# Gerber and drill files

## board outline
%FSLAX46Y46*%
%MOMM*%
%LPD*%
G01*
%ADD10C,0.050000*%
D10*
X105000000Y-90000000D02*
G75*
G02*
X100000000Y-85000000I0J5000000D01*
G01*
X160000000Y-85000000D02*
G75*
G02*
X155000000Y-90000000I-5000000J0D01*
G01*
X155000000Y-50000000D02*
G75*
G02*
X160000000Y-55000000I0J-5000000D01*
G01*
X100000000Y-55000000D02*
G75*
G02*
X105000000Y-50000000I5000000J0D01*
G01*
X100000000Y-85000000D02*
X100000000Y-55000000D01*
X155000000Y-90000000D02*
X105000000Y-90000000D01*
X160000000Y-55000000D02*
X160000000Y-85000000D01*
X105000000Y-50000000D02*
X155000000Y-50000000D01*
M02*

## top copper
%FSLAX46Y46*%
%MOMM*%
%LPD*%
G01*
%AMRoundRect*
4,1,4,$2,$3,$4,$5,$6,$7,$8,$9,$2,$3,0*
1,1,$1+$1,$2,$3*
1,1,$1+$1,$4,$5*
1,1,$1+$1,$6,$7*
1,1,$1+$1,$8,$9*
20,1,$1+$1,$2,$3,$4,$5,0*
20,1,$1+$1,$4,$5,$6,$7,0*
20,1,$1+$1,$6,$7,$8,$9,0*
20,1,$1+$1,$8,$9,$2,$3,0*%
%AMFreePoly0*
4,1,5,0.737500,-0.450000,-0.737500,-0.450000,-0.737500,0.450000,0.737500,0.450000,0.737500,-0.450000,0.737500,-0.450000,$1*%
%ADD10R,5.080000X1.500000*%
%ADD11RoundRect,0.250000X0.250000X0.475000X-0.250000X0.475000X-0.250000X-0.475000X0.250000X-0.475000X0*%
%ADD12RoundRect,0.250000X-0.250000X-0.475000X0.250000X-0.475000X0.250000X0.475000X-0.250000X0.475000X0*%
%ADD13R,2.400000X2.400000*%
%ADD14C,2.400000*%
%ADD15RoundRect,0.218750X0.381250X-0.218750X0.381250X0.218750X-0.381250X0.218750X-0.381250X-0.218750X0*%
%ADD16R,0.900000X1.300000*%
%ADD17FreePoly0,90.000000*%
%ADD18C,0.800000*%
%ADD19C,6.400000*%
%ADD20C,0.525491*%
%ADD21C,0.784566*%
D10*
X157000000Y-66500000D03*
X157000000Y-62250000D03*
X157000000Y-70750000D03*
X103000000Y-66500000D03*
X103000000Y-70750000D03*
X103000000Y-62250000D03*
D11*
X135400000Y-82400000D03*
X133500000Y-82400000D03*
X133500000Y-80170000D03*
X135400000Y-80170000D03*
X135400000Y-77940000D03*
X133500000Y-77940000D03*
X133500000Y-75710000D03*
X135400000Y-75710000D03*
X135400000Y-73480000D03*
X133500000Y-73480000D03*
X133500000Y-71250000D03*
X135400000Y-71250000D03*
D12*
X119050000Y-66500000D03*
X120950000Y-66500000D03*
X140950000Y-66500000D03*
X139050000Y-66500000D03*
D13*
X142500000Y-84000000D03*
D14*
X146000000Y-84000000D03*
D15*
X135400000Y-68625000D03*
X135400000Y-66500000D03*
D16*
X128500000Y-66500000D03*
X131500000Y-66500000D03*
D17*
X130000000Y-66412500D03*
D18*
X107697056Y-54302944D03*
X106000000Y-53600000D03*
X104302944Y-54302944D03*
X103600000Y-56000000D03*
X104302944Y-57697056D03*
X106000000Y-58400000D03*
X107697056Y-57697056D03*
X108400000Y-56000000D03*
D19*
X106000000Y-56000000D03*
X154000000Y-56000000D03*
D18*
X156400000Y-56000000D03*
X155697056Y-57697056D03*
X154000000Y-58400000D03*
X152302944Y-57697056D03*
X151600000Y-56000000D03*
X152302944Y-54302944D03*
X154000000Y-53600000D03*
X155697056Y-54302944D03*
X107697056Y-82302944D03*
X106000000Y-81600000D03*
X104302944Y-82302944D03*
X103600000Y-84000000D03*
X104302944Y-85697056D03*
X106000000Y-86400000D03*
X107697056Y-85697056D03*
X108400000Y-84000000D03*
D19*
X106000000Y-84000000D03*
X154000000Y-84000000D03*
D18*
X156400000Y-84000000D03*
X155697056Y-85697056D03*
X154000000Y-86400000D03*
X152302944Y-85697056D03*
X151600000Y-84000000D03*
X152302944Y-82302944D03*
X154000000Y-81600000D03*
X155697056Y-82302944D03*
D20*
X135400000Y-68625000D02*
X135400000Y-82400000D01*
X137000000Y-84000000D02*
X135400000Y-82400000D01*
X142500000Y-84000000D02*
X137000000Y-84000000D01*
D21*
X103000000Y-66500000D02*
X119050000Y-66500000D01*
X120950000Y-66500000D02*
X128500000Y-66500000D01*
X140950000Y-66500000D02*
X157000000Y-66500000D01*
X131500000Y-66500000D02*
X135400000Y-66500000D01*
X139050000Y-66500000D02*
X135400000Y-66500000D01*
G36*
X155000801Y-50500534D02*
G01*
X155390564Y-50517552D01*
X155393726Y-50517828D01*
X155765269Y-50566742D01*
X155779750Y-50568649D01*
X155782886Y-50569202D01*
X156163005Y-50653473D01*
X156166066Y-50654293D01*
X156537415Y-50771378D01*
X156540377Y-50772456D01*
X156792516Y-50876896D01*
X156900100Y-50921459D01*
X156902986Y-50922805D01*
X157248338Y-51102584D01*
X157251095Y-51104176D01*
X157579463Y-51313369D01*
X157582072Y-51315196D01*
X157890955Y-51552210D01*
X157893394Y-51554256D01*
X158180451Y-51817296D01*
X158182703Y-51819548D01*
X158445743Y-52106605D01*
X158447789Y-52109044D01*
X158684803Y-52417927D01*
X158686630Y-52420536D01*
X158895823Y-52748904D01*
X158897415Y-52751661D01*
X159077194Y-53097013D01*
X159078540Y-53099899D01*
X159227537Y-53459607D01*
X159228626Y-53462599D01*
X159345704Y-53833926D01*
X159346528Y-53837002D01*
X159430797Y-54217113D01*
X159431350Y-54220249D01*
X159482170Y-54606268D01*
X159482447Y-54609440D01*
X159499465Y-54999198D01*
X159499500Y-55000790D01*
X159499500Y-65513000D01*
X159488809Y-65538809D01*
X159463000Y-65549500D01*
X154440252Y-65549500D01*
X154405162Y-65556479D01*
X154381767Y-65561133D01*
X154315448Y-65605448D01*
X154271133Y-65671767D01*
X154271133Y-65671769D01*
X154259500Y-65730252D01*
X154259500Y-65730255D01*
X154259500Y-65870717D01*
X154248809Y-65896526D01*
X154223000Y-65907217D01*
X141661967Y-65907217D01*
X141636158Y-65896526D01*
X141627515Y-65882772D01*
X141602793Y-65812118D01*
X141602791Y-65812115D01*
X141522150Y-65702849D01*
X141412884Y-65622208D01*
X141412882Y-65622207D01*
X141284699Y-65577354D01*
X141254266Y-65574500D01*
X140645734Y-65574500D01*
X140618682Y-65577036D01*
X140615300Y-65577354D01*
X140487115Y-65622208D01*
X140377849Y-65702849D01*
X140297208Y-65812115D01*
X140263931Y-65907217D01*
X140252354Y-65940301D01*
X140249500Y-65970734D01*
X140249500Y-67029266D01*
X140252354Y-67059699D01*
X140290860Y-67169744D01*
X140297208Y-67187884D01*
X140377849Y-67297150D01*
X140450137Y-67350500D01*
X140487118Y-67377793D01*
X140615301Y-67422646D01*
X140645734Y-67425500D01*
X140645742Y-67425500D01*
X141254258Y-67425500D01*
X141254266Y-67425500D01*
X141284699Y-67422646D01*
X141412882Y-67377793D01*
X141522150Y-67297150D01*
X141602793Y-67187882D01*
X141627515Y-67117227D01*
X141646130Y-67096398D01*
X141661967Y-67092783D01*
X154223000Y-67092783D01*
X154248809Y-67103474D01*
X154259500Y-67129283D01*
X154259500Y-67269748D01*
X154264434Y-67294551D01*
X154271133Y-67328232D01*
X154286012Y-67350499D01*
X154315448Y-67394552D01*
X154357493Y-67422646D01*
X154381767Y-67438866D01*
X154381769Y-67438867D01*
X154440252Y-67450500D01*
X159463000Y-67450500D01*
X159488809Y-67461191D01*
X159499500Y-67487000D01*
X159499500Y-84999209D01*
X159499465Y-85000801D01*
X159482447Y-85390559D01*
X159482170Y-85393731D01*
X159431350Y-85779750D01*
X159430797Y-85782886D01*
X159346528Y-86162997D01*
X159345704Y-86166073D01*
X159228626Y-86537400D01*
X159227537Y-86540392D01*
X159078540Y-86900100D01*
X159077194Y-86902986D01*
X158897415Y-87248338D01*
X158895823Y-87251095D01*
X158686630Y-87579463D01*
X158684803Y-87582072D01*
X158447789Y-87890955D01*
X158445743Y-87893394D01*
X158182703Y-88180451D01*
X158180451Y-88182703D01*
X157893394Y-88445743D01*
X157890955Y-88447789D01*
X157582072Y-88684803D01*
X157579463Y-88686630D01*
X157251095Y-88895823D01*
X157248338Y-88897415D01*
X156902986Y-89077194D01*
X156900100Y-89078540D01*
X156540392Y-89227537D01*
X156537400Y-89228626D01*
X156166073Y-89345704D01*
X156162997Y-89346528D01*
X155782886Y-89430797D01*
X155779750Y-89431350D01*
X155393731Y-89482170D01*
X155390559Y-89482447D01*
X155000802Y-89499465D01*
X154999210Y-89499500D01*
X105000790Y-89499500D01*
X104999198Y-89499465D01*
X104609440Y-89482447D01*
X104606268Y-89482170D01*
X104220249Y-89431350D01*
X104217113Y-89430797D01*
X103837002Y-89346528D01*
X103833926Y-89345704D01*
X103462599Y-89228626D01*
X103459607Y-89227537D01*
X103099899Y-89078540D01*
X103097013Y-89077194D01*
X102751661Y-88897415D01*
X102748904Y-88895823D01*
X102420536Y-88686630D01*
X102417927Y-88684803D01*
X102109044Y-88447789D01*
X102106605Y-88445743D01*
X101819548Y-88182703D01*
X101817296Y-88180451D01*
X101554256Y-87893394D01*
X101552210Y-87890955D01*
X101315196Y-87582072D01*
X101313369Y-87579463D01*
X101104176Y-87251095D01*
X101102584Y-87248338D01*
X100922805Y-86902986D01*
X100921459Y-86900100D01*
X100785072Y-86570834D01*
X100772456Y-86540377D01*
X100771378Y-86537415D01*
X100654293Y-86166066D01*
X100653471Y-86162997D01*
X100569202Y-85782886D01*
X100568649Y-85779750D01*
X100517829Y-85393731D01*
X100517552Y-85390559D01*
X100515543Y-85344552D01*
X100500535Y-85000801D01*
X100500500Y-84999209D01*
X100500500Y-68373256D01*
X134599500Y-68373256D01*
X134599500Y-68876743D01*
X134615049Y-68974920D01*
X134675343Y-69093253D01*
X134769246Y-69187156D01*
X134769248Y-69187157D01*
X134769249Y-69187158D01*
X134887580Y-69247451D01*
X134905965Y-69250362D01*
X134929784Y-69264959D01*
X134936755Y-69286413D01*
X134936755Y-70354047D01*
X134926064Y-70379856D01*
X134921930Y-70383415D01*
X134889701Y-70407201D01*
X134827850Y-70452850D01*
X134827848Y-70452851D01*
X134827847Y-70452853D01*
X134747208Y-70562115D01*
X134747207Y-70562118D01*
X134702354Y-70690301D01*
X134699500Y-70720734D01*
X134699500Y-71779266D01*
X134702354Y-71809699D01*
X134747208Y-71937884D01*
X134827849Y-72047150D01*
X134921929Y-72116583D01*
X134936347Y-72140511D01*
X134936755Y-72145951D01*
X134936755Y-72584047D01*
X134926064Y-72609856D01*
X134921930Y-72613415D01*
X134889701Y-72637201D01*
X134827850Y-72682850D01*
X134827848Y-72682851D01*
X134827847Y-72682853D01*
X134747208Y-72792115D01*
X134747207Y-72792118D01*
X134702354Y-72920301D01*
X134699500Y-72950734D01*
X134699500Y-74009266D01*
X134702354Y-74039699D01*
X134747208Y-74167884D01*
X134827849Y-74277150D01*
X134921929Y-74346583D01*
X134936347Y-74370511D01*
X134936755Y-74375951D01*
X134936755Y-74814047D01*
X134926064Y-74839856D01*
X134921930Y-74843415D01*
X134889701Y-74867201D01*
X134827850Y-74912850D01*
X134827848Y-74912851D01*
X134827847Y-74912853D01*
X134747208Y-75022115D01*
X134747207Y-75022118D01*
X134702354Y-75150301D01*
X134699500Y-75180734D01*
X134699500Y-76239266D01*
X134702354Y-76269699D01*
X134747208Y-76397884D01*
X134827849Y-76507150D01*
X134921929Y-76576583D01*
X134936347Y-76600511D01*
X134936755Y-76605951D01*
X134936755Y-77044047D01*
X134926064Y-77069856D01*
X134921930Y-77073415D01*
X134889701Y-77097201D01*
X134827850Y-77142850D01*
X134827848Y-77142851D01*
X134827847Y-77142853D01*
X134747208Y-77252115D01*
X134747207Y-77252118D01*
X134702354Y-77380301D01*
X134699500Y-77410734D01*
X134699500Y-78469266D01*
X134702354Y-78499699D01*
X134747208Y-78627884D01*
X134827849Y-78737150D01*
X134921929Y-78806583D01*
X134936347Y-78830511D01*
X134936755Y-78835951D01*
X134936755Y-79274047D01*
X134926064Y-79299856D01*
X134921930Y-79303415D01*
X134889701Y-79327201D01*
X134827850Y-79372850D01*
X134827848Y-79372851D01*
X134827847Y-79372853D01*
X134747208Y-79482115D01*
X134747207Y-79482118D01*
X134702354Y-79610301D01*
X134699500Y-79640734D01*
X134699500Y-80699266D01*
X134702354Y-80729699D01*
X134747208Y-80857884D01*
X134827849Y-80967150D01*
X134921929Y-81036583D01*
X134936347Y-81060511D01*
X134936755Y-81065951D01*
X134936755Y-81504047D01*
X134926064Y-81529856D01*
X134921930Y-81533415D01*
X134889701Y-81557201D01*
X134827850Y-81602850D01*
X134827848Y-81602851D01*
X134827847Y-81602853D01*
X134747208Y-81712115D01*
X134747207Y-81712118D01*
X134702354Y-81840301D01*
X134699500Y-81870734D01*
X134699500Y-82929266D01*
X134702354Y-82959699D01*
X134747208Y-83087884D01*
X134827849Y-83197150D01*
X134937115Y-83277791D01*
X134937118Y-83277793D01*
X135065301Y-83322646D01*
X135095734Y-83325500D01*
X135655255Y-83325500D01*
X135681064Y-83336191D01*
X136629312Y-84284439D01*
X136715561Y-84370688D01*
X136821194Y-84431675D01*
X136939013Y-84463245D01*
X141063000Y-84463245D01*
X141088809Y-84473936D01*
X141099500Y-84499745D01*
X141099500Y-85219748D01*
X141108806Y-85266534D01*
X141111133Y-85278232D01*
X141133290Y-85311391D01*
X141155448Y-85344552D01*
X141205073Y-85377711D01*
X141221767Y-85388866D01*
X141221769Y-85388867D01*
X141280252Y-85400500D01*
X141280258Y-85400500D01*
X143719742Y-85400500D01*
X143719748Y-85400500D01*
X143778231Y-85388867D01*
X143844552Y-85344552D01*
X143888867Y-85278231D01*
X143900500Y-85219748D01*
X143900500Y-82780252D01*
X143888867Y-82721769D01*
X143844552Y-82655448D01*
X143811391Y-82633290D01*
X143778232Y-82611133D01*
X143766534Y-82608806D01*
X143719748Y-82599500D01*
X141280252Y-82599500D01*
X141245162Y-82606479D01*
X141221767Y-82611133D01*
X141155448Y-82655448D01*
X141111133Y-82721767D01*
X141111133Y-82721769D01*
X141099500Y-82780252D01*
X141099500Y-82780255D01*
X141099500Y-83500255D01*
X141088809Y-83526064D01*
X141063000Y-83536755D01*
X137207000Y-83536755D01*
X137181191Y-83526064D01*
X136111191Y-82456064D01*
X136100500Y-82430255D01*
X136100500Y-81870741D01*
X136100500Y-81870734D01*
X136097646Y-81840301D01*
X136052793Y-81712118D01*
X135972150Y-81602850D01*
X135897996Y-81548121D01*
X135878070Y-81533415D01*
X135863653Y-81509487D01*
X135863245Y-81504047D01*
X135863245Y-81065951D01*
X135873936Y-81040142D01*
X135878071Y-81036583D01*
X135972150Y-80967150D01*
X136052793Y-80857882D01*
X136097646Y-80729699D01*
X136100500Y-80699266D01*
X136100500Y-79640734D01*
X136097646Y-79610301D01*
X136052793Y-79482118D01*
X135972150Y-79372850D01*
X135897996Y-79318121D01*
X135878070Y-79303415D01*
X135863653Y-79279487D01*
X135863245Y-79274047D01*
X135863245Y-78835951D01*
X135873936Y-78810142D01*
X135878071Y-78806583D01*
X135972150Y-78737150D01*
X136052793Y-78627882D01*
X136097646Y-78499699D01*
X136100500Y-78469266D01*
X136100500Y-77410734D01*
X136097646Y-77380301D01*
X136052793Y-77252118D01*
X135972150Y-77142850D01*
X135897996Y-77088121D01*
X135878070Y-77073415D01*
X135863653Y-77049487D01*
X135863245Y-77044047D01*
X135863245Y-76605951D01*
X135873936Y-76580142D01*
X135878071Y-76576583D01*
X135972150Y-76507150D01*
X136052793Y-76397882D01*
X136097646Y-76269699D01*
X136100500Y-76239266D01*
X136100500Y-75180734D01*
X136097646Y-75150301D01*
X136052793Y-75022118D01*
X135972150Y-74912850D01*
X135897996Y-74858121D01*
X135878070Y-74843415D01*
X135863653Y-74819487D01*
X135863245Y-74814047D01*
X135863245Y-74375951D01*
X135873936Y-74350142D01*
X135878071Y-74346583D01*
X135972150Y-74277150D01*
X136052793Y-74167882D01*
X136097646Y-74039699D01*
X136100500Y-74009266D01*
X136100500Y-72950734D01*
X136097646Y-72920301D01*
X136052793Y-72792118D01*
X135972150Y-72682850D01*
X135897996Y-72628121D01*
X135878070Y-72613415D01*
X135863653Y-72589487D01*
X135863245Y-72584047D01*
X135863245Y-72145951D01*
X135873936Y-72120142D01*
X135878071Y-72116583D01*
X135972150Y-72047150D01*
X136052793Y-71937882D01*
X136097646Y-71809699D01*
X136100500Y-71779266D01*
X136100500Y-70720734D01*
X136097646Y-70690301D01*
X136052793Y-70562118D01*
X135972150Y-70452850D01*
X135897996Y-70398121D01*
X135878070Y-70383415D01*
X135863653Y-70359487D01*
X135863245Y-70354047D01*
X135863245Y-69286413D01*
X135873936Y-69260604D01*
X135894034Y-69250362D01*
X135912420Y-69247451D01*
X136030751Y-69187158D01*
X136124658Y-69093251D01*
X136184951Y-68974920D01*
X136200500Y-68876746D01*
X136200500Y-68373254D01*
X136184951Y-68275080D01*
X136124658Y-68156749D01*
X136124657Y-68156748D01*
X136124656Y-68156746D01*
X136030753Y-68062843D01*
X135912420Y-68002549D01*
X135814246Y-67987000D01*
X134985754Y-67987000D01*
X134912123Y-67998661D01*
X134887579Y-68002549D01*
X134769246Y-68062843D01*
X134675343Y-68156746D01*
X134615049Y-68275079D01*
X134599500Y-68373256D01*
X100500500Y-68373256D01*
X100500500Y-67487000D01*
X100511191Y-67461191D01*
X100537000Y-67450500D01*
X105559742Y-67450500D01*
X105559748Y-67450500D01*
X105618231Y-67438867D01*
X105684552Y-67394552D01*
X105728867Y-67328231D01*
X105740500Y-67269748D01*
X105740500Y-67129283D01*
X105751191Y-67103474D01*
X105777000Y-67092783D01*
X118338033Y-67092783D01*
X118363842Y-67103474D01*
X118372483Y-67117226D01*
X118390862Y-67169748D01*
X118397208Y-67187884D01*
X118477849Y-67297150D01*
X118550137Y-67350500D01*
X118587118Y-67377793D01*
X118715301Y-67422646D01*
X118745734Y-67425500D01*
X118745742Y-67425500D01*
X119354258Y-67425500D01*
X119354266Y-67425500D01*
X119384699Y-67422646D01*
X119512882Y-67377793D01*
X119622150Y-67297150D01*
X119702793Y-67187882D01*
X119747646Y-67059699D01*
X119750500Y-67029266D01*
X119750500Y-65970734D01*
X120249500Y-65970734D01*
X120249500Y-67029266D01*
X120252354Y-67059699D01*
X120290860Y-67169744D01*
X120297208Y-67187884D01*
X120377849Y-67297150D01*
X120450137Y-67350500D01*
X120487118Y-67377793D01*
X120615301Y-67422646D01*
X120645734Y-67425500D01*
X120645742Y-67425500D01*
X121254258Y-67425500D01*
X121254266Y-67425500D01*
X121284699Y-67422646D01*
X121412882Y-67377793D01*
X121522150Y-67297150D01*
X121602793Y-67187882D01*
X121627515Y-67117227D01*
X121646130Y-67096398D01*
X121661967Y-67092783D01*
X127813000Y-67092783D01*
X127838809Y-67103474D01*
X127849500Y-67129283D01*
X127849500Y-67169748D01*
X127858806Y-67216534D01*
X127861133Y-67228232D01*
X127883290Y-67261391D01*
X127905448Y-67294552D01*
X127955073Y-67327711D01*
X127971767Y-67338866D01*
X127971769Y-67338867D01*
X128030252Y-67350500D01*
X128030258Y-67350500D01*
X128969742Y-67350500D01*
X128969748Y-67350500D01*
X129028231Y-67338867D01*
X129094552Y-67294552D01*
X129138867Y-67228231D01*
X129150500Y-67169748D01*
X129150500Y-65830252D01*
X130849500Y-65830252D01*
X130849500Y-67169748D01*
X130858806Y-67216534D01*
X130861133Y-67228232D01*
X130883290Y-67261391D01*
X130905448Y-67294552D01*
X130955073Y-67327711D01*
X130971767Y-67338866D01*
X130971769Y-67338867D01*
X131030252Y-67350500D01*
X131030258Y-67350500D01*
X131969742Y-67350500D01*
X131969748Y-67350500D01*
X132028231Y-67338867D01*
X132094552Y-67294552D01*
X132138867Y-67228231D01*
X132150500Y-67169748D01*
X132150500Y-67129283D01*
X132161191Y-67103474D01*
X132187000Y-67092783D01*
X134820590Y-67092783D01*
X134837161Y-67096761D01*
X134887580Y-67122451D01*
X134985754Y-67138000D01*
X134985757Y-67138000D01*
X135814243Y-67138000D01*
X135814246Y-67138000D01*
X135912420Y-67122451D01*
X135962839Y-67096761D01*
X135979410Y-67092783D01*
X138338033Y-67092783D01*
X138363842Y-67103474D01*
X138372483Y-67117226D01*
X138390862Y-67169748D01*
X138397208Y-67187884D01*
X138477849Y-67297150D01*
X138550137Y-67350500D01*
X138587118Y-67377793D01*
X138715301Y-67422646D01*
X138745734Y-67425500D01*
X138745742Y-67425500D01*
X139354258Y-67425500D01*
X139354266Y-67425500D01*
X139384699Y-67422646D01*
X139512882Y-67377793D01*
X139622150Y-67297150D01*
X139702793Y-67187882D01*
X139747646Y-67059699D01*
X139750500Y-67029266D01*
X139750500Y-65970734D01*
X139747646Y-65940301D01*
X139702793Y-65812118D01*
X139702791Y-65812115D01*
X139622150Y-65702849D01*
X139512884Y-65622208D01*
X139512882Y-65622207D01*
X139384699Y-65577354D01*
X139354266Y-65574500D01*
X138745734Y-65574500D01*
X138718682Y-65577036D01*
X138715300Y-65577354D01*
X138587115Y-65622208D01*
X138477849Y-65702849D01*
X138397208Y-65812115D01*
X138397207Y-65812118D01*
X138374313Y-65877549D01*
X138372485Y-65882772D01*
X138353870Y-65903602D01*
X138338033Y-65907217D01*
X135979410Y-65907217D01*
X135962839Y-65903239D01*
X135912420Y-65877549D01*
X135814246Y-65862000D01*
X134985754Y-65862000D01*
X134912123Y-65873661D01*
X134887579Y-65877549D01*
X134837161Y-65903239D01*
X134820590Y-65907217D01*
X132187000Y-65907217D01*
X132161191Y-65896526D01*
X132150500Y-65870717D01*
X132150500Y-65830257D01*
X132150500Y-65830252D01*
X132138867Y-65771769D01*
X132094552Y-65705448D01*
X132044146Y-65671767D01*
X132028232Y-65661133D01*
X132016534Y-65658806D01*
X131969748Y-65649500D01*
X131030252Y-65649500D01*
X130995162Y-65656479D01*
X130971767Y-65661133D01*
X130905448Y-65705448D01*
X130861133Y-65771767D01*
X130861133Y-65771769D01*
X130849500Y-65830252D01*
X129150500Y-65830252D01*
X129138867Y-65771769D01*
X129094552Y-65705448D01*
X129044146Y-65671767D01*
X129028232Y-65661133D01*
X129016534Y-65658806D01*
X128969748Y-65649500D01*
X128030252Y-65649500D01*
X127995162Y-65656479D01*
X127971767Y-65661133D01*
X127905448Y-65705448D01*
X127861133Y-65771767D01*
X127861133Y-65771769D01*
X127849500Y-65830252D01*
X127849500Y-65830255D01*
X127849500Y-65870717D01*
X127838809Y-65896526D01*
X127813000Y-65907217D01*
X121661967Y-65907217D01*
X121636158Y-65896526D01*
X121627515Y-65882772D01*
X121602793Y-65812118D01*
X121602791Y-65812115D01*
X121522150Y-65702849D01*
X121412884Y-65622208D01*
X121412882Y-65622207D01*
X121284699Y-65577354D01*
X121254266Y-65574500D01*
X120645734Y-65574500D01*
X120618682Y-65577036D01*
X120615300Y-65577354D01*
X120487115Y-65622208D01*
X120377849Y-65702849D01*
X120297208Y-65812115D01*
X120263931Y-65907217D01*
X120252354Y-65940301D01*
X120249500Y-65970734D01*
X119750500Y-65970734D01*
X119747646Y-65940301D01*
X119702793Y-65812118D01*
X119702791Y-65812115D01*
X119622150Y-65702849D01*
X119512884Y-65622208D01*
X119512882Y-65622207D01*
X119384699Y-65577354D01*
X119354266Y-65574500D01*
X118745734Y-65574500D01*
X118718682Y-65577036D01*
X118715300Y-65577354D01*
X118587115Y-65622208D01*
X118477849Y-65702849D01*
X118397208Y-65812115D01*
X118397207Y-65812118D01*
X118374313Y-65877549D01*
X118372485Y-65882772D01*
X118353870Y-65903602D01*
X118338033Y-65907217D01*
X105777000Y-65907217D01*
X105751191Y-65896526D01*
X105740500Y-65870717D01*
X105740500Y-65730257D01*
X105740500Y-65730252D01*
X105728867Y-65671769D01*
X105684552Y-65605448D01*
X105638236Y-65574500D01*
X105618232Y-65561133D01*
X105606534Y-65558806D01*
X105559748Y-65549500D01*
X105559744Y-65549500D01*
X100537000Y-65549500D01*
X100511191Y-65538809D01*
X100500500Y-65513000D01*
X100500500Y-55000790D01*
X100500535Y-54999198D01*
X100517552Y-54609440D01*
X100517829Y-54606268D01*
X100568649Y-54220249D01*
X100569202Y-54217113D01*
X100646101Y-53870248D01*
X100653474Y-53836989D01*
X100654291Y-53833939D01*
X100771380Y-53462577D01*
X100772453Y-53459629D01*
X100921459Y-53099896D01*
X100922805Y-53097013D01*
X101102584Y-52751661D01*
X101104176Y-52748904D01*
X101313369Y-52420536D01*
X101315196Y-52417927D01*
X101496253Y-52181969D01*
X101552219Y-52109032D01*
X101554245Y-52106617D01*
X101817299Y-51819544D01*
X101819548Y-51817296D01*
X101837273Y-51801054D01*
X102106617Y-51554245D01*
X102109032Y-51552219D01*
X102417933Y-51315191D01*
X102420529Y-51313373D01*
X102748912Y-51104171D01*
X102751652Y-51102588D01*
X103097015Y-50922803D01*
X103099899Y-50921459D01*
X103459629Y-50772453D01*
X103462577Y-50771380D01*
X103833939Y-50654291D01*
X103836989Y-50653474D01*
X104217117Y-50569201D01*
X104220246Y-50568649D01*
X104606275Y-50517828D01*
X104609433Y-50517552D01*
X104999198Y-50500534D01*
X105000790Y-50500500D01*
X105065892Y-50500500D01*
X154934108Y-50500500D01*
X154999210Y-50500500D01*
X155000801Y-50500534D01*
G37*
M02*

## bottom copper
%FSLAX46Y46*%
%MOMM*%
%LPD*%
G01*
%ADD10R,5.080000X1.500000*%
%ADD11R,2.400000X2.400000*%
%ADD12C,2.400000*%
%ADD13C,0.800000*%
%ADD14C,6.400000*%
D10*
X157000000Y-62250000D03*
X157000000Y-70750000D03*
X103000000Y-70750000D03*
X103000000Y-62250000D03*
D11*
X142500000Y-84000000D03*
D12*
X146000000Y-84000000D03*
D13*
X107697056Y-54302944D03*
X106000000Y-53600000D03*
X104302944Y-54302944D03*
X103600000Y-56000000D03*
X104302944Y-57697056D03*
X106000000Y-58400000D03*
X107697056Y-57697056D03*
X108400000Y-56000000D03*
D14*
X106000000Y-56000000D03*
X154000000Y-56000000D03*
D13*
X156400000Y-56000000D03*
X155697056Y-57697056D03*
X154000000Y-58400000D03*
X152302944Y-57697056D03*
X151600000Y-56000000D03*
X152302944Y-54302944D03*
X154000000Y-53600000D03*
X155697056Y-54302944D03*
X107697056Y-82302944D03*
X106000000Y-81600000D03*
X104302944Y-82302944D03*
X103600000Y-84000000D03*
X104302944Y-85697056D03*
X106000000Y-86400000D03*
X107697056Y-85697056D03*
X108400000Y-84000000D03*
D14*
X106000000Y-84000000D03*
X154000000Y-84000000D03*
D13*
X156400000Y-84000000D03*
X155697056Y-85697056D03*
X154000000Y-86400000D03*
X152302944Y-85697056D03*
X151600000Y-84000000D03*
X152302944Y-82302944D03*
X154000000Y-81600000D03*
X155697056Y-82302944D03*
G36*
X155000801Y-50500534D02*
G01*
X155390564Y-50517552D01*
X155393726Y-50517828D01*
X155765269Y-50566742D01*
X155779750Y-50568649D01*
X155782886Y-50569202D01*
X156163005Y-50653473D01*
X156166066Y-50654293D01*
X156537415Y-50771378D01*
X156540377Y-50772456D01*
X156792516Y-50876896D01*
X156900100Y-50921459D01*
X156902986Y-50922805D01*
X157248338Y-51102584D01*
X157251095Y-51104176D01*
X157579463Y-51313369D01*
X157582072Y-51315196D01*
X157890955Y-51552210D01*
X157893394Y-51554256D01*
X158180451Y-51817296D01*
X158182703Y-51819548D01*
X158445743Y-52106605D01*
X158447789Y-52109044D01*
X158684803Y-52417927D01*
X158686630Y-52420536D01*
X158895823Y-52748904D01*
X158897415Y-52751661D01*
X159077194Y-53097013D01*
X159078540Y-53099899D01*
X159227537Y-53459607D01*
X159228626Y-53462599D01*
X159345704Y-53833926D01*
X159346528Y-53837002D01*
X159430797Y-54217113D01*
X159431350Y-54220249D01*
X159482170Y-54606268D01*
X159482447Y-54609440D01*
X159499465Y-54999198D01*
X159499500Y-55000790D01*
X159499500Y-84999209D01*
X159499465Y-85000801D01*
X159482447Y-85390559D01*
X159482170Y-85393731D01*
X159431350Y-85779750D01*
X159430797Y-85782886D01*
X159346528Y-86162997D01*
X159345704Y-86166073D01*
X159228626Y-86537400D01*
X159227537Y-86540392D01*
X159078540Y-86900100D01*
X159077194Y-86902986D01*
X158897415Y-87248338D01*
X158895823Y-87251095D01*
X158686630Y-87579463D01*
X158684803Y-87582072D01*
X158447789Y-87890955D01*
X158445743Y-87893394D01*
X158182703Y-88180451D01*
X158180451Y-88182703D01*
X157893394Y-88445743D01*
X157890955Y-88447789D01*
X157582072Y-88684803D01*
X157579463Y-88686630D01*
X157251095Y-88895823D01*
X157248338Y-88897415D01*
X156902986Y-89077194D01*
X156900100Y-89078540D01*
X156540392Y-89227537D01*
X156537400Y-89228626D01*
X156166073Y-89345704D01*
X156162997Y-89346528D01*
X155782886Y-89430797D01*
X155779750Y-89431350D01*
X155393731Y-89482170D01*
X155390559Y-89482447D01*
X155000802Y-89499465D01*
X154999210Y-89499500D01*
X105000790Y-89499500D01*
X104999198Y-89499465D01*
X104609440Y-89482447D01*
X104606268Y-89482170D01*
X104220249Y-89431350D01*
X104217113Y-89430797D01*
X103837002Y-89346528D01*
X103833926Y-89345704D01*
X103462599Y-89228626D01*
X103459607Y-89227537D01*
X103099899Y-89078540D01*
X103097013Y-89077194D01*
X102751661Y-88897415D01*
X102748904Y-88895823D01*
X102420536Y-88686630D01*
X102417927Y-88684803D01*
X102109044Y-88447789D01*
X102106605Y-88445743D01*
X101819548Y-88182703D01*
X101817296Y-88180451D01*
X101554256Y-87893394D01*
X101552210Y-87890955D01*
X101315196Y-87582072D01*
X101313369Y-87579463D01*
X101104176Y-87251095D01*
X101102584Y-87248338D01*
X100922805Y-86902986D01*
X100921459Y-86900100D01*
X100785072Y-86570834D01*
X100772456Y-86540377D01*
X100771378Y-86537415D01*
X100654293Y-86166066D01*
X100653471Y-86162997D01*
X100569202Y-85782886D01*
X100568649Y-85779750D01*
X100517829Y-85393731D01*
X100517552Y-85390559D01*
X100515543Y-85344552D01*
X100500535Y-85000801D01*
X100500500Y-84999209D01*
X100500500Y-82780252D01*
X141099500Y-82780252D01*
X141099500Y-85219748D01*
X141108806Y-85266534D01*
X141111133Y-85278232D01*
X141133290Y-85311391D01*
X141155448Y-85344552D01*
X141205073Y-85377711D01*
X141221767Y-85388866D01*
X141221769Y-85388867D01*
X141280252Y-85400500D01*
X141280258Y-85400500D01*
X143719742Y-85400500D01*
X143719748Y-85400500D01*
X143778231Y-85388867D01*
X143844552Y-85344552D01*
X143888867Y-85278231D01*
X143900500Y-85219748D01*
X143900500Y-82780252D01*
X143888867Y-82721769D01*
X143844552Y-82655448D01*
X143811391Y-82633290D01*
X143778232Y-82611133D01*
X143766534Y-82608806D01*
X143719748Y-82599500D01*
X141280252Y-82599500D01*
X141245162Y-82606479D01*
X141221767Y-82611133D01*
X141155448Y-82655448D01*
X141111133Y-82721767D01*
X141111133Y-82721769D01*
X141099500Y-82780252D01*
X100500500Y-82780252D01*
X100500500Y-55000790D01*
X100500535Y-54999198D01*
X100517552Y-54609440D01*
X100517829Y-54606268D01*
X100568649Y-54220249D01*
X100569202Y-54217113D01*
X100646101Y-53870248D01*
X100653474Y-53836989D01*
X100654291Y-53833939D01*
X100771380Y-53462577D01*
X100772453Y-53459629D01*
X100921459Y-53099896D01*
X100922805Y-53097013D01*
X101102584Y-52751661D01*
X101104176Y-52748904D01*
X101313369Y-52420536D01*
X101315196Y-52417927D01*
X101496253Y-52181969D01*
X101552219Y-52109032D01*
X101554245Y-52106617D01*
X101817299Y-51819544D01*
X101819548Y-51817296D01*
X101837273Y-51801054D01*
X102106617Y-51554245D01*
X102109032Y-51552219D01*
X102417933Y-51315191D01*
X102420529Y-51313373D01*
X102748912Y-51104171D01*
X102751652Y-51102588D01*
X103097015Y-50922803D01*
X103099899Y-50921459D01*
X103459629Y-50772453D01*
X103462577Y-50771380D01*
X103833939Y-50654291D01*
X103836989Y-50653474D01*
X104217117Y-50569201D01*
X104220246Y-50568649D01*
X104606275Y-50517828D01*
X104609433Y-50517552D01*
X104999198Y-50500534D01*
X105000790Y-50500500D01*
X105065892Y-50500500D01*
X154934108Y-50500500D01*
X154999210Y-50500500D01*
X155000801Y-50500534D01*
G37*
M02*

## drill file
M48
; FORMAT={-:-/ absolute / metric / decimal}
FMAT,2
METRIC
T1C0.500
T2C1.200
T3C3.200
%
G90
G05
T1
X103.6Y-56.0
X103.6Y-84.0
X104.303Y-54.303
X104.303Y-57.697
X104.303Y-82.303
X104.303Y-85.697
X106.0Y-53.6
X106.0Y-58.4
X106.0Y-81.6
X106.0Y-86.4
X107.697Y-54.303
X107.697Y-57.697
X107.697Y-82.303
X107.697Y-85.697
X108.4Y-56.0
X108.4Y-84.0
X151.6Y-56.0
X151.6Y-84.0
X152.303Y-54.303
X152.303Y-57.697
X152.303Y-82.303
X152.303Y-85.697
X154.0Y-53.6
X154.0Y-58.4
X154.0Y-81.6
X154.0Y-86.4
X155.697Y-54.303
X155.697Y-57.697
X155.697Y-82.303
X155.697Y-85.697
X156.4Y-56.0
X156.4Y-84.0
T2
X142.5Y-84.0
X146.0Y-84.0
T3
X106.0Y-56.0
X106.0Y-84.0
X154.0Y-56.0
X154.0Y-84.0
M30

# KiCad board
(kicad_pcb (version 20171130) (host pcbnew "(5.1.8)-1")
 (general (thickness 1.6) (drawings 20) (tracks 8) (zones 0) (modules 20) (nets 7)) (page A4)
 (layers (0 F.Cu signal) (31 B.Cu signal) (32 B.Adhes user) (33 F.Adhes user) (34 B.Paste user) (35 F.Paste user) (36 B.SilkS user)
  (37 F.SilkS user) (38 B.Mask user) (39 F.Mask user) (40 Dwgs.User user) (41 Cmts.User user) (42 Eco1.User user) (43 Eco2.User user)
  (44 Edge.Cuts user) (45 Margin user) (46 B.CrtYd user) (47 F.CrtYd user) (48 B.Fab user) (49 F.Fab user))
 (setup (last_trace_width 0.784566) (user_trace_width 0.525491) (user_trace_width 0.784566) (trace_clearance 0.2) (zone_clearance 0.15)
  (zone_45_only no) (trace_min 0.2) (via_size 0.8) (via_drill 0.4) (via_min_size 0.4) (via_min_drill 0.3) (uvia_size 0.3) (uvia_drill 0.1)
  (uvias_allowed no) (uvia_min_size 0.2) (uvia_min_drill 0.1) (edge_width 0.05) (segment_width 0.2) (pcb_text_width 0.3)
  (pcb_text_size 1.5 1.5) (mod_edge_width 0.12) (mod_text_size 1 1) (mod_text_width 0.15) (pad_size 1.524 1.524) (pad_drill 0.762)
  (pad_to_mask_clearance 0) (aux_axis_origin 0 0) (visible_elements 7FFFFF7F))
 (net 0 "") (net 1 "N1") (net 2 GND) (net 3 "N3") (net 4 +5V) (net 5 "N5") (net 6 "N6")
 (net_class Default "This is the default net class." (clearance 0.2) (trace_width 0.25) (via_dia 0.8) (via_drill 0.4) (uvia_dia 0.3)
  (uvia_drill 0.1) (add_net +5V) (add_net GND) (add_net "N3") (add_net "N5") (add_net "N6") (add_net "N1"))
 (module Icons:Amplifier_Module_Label (layer F.Cu) (at 130 55.99889)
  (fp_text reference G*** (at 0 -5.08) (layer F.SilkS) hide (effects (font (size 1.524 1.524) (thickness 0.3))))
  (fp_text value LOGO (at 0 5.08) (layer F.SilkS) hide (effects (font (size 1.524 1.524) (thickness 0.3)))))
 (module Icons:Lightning (layer F.Cu) (at 144.25 78.5)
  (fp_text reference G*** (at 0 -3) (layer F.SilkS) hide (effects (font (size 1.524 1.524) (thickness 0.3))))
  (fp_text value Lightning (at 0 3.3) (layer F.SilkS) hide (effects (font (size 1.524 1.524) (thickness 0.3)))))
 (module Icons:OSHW (layer F.Cu) (at 116 75)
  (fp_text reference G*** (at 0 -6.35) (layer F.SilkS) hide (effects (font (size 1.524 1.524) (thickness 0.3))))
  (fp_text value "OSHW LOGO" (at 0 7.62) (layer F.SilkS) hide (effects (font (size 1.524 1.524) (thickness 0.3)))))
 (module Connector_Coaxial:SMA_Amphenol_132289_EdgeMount (layer F.Cu) (at 157 66.5)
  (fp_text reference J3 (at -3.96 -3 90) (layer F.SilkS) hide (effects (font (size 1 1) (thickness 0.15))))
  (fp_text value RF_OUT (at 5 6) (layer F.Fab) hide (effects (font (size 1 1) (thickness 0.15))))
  (pad 1 smd rect (at 0 0 90) (size 1.5 5.08) (layers F.Cu F.Paste F.Mask) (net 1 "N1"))
  (pad 2 smd rect (at 0 -4.25 90) (size 1.5 5.08) (layers F.Cu F.Paste F.Mask) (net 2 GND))
  (pad 2 smd rect (at 0 4.25 90) (size 1.5 5.08) (layers F.Cu F.Paste F.Mask) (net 2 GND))
  (pad 2 smd rect (at 0 -4.25 90) (size 1.5 5.08) (layers B.Cu B.Paste B.Mask) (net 2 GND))
  (pad 2 smd rect (at 0 4.25 90) (size 1.5 5.08) (layers B.Cu B.Paste B.Mask) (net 2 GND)))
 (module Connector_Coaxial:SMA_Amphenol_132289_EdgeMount (layer F.Cu) (at 103 66.5 180)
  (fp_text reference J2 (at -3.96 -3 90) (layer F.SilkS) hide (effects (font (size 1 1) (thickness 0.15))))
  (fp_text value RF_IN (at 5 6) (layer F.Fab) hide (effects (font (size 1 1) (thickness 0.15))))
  (pad 1 smd rect (at 0 0 270) (size 1.5 5.08) (layers F.Cu F.Paste F.Mask) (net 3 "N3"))
  (pad 2 smd rect (at 0 -4.25 270) (size 1.5 5.08) (layers F.Cu F.Paste F.Mask) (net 2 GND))
  (pad 2 smd rect (at 0 4.25 270) (size 1.5 5.08) (layers F.Cu F.Paste F.Mask) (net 2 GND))
  (pad 2 smd rect (at 0 -4.25 270) (size 1.5 5.08) (layers B.Cu B.Paste B.Mask) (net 2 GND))
  (pad 2 smd rect (at 0 4.25 270) (size 1.5 5.08) (layers B.Cu B.Paste B.Mask) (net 2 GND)))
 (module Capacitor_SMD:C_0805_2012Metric (layer F.Cu) (at 134.45 82.4 180)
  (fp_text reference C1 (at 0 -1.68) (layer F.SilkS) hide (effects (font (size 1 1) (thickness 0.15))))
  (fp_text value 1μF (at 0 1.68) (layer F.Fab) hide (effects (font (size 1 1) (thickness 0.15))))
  (pad 1 smd roundrect (at -0.95 0 180) (size 1 1.45) (layers F.Cu F.Paste F.Mask) (roundrect_rratio 0.25) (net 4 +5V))
  (pad 2 smd roundrect (at 0.95 0 180) (size 1 1.45) (layers F.Cu F.Paste F.Mask) (roundrect_rratio 0.25) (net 2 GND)))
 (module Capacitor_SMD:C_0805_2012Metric (layer F.Cu) (at 134.45 80.17 180)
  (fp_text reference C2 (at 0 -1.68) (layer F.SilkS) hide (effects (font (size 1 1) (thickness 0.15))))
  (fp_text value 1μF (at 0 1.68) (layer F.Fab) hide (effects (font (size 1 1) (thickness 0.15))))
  (pad 2 smd roundrect (at 0.95 0 180) (size 1 1.45) (layers F.Cu F.Paste F.Mask) (roundrect_rratio 0.25) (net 2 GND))
  (pad 1 smd roundrect (at -0.95 0 180) (size 1 1.45) (layers F.Cu F.Paste F.Mask) (roundrect_rratio 0.25) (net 4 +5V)))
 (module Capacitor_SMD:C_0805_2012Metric (layer F.Cu) (at 134.45 77.94 180)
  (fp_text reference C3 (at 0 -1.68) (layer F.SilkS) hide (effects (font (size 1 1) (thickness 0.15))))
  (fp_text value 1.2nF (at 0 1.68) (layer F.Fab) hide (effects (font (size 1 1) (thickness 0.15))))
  (pad 1 smd roundrect (at -0.95 0 180) (size 1 1.45) (layers F.Cu F.Paste F.Mask) (roundrect_rratio 0.25) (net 4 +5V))
  (pad 2 smd roundrect (at 0.95 0 180) (size 1 1.45) (layers F.Cu F.Paste F.Mask) (roundrect_rratio 0.25) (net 2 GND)))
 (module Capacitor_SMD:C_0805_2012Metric (layer F.Cu) (at 134.45 75.71 180)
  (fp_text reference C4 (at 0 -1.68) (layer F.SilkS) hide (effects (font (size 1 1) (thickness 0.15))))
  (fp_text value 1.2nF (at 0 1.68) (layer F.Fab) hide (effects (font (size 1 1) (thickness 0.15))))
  (pad 2 smd roundrect (at 0.95 0 180) (size 1 1.45) (layers F.Cu F.Paste F.Mask) (roundrect_rratio 0.25) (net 2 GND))
  (pad 1 smd roundrect (at -0.95 0 180) (size 1 1.45) (layers F.Cu F.Paste F.Mask) (roundrect_rratio 0.25) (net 4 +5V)))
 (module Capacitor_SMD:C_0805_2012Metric (layer F.Cu) (at 134.45 73.48 180)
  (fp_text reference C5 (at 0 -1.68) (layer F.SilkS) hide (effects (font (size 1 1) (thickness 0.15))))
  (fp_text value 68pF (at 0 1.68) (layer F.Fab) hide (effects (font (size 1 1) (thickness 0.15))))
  (pad 1 smd roundrect (at -0.95 0 180) (size 1 1.45) (layers F.Cu F.Paste F.Mask) (roundrect_rratio 0.25) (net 4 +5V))
  (pad 2 smd roundrect (at 0.95 0 180) (size 1 1.45) (layers F.Cu F.Paste F.Mask) (roundrect_rratio 0.25) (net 2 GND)))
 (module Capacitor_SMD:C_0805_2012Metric (layer F.Cu) (at 134.45 71.25 180)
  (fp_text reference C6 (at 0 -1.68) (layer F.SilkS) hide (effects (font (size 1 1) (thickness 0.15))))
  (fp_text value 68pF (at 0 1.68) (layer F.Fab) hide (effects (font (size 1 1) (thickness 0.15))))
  (pad 2 smd roundrect (at 0.95 0 180) (size 1 1.45) (layers F.Cu F.Paste F.Mask) (roundrect_rratio 0.25) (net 2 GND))
  (pad 1 smd roundrect (at -0.95 0 180) (size 1 1.45) (layers F.Cu F.Paste F.Mask) (roundrect_rratio 0.25) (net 4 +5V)))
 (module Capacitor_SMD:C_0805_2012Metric (layer F.Cu) (at 120 66.5)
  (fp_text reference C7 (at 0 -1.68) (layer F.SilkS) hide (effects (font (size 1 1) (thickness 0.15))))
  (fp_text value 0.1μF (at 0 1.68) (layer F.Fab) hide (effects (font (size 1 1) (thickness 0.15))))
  (pad 1 smd roundrect (at -0.95 0) (size 1 1.45) (layers F.Cu F.Paste F.Mask) (roundrect_rratio 0.25) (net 3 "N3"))
  (pad 2 smd roundrect (at 0.95 0) (size 1 1.45) (layers F.Cu F.Paste F.Mask) (roundrect_rratio 0.25) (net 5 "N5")))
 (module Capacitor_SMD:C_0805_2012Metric (layer F.Cu) (at 140 66.5)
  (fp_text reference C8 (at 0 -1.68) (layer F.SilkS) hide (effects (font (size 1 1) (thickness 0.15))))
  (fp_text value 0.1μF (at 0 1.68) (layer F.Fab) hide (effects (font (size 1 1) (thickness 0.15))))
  (pad 2 smd roundrect (at 0.95 0) (size 1 1.45) (layers F.Cu F.Paste F.Mask) (roundrect_rratio 0.25) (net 1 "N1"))
  (pad 1 smd roundrect (at -0.95 0) (size 1 1.45) (layers F.Cu F.Paste F.Mask) (roundrect_rratio 0.25) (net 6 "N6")))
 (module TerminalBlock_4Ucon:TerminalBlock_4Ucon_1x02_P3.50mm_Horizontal (layer F.Cu) (at 142.5 84)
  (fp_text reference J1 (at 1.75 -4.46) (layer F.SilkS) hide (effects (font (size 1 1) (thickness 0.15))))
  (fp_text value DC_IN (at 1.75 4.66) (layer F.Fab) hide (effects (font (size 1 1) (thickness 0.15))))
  (pad 1 thru_hole rect (at 0 0) (size 2.4 2.4) (drill 1.2) (layers *.Cu *.Mask) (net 4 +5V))
  (pad 2 thru_hole circle (at 3.5 0) (size 2.4 2.4) (drill 1.2) (layers *.Cu *.Mask) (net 2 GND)))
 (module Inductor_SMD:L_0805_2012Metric (layer F.Cu) (at 135.4 67.5625 90)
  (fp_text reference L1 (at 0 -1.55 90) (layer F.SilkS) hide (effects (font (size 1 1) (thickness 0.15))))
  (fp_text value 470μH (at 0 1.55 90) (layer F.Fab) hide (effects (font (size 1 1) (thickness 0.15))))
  (pad 1 smd roundrect (at -1.0625 0 90) (size 0.875 1.2) (layers F.Cu F.Paste F.Mask) (roundrect_rratio 0.25) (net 4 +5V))
  (pad 2 smd roundrect (at 1.0625 0 90) (size 0.875 1.2) (layers F.Cu F.Paste F.Mask) (roundrect_rratio 0.25) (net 6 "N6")))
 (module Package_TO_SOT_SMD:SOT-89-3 (layer F.Cu) (at 130 64.85 90)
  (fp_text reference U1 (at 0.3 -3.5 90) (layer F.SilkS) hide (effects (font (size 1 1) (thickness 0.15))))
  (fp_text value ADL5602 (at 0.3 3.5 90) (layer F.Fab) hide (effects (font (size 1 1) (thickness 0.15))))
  (pad 1 smd rect (at -1.65 -1.5 90) (size 1.3 0.9) (layers F.Cu F.Paste F.Mask) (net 5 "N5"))
  (pad 3 smd rect (at -1.65 1.5 90) (size 1.3 0.9) (layers F.Cu F.Paste F.Mask) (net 6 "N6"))
  (pad 2 smd custom (at -1.5625 0 90) (size 1.475 0.9) (layers F.Cu F.Paste F.Mask) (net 2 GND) (zone_connect 2)
   (options (clearance outline) (anchor rect)) (primitives)))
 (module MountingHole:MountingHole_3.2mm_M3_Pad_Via (layer F.Cu) (at 106 56)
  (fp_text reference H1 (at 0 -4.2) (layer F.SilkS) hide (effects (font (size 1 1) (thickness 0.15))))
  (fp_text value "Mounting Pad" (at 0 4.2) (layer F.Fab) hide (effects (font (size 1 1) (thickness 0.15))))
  (pad 1 thru_hole circle (at 1.697056 -1.697056) (size 0.8 0.8) (drill 0.5) (layers *.Cu *.Mask) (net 2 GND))
  (pad 1 thru_hole circle (at 0 -2.4) (size 0.8 0.8) (drill 0.5) (layers *.Cu *.Mask) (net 2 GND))
  (pad 1 thru_hole circle (at -1.697056 -1.697056) (size 0.8 0.8) (drill 0.5) (layers *.Cu *.Mask) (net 2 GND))
  (pad 1 thru_hole circle (at -2.4 0) (size 0.8 0.8) (drill 0.5) (layers *.Cu *.Mask) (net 2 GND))
  (pad 1 thru_hole circle (at -1.697056 1.697056) (size 0.8 0.8) (drill 0.5) (layers *.Cu *.Mask) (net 2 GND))
  (pad 1 thru_hole circle (at 0 2.4) (size 0.8 0.8) (drill 0.5) (layers *.Cu *.Mask) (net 2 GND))
  (pad 1 thru_hole circle (at 1.697056 1.697056) (size 0.8 0.8) (drill 0.5) (layers *.Cu *.Mask) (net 2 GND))
  (pad 1 thru_hole circle (at 2.4 0) (size 0.8 0.8) (drill 0.5) (layers *.Cu *.Mask) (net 2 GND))
  (pad 1 thru_hole circle (at 0 0) (size 6.4 6.4) (drill 3.2) (layers *.Cu *.Mask) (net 2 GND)))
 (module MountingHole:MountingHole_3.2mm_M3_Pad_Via (layer F.Cu) (at 154 56)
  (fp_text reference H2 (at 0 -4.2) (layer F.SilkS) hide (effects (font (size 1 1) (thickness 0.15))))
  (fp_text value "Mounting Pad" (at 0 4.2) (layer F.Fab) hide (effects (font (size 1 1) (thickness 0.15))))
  (pad 1 thru_hole circle (at 0 0) (size 6.4 6.4) (drill 3.2) (layers *.Cu *.Mask) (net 2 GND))
  (pad 1 thru_hole circle (at 2.4 0) (size 0.8 0.8) (drill 0.5) (layers *.Cu *.Mask) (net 2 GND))
  (pad 1 thru_hole circle (at 1.697056 1.697056) (size 0.8 0.8) (drill 0.5) (layers *.Cu *.Mask) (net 2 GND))
  (pad 1 thru_hole circle (at 0 2.4) (size 0.8 0.8) (drill 0.5) (layers *.Cu *.Mask) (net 2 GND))
  (pad 1 thru_hole circle (at -1.697056 1.697056) (size 0.8 0.8) (drill 0.5) (layers *.Cu *.Mask) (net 2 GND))
  (pad 1 thru_hole circle (at -2.4 0) (size 0.8 0.8) (drill 0.5) (layers *.Cu *.Mask) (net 2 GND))
  (pad 1 thru_hole circle (at -1.697056 -1.697056) (size 0.8 0.8) (drill 0.5) (layers *.Cu *.Mask) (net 2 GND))
  (pad 1 thru_hole circle (at 0 -2.4) (size 0.8 0.8) (drill 0.5) (layers *.Cu *.Mask) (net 2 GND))
  (pad 1 thru_hole circle (at 1.697056 -1.697056) (size 0.8 0.8) (drill 0.5) (layers *.Cu *.Mask) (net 2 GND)))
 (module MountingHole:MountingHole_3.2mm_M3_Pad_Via (layer F.Cu) (at 106 84)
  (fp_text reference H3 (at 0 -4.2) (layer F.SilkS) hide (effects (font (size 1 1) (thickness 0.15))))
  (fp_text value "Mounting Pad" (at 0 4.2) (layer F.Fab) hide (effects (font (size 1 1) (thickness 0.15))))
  (pad 1 thru_hole circle (at 1.697056 -1.697056) (size 0.8 0.8) (drill 0.5) (layers *.Cu *.Mask) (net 2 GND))
  (pad 1 thru_hole circle (at 0 -2.4) (size 0.8 0.8) (drill 0.5) (layers *.Cu *.Mask) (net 2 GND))
  (pad 1 thru_hole circle (at -1.697056 -1.697056) (size 0.8 0.8) (drill 0.5) (layers *.Cu *.Mask) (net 2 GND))
  (pad 1 thru_hole circle (at -2.4 0) (size 0.8 0.8) (drill 0.5) (layers *.Cu *.Mask) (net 2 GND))
  (pad 1 thru_hole circle (at -1.697056 1.697056) (size 0.8 0.8) (drill 0.5) (layers *.Cu *.Mask) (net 2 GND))
  (pad 1 thru_hole circle (at 0 2.4) (size 0.8 0.8) (drill 0.5) (layers *.Cu *.Mask) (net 2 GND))
  (pad 1 thru_hole circle (at 1.697056 1.697056) (size 0.8 0.8) (drill 0.5) (layers *.Cu *.Mask) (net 2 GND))
  (pad 1 thru_hole circle (at 2.4 0) (size 0.8 0.8) (drill 0.5) (layers *.Cu *.Mask) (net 2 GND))
  (pad 1 thru_hole circle (at 0 0) (size 6.4 6.4) (drill 3.2) (layers *.Cu *.Mask) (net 2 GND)))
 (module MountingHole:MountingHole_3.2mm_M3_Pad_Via (layer F.Cu) (at 154 84)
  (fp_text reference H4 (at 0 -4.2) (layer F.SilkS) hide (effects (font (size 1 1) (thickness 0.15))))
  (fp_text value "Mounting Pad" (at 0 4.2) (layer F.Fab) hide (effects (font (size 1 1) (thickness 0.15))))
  (pad 1 thru_hole circle (at 0 0) (size 6.4 6.4) (drill 3.2) (layers *.Cu *.Mask) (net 2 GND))
  (pad 1 thru_hole circle (at 2.4 0) (size 0.8 0.8) (drill 0.5) (layers *.Cu *.Mask) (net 2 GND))
  (pad 1 thru_hole circle (at 1.697056 1.697056) (size 0.8 0.8) (drill 0.5) (layers *.Cu *.Mask) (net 2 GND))
  (pad 1 thru_hole circle (at 0 2.4) (size 0.8 0.8) (drill 0.5) (layers *.Cu *.Mask) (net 2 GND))
  (pad 1 thru_hole circle (at -1.697056 1.697056) (size 0.8 0.8) (drill 0.5) (layers *.Cu *.Mask) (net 2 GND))
  (pad 1 thru_hole circle (at -2.4 0) (size 0.8 0.8) (drill 0.5) (layers *.Cu *.Mask) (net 2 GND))
  (pad 1 thru_hole circle (at -1.697056 -1.697056) (size 0.8 0.8) (drill 0.5) (layers *.Cu *.Mask) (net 2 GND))
  (pad 1 thru_hole circle (at 0 -2.4) (size 0.8 0.8) (drill 0.5) (layers *.Cu *.Mask) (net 2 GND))
  (pad 1 thru_hole circle (at 1.697056 -1.697056) (size 0.8 0.8) (drill 0.5) (layers *.Cu *.Mask) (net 2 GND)))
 (gr_arc (start 105 85) (end 100 85) (angle -90) (layer Edge.Cuts) (width 0.05))
 (gr_arc (start 155 85) (end 155 90) (angle -90) (layer Edge.Cuts) (width 0.05))
 (gr_arc (start 155 55) (end 160 55) (angle -90) (layer Edge.Cuts) (width 0.05))
 (gr_arc (start 105 55) (end 105 50) (angle -90) (layer Edge.Cuts) (width 0.05))
 (gr_line (start 100 85) (end 100 55) (layer Edge.Cuts) (width 0.05))
 (gr_line (start 155 90) (end 105 90) (layer Edge.Cuts) (width 0.05))
 (gr_line (start 160 55) (end 160 85) (layer Edge.Cuts) (width 0.05))
 (gr_line (start 105 50) (end 155 50) (layer Edge.Cuts) (width 0.05))
 (segment (start 135.4 68.625) (end 135.4 82.4) (width 0.525491) (layer F.Cu) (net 4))
 (segment (start 137 84) (end 135.4 82.4) (width 0.525491) (layer F.Cu) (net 4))
 (segment (start 142.5 84) (end 137 84) (width 0.525491) (layer F.Cu) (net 4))
 (segment (start 103 66.5) (end 119.05 66.5) (width 0.784566) (layer F.Cu) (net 3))
 (segment (start 120.95 66.5) (end 128.5 66.5) (width 0.784566) (layer F.Cu) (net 5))
 (segment (start 140.95 66.5) (end 157 66.5) (width 0.784566) (layer F.Cu) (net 1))
 (segment (start 131.5 66.5) (end 135.4 66.5) (width 0.784566) (layer F.Cu) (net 6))
 (segment (start 139.05 66.5) (end 135.4 66.5) (width 0.784566) (layer F.Cu) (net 6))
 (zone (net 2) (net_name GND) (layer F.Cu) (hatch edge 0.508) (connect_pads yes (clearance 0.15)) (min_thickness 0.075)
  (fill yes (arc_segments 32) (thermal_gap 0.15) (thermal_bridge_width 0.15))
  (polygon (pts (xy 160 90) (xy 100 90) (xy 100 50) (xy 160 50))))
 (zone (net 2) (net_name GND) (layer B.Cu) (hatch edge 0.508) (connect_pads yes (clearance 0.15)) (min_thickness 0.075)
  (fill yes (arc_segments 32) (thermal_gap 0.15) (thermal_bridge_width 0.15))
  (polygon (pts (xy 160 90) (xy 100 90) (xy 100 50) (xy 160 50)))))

